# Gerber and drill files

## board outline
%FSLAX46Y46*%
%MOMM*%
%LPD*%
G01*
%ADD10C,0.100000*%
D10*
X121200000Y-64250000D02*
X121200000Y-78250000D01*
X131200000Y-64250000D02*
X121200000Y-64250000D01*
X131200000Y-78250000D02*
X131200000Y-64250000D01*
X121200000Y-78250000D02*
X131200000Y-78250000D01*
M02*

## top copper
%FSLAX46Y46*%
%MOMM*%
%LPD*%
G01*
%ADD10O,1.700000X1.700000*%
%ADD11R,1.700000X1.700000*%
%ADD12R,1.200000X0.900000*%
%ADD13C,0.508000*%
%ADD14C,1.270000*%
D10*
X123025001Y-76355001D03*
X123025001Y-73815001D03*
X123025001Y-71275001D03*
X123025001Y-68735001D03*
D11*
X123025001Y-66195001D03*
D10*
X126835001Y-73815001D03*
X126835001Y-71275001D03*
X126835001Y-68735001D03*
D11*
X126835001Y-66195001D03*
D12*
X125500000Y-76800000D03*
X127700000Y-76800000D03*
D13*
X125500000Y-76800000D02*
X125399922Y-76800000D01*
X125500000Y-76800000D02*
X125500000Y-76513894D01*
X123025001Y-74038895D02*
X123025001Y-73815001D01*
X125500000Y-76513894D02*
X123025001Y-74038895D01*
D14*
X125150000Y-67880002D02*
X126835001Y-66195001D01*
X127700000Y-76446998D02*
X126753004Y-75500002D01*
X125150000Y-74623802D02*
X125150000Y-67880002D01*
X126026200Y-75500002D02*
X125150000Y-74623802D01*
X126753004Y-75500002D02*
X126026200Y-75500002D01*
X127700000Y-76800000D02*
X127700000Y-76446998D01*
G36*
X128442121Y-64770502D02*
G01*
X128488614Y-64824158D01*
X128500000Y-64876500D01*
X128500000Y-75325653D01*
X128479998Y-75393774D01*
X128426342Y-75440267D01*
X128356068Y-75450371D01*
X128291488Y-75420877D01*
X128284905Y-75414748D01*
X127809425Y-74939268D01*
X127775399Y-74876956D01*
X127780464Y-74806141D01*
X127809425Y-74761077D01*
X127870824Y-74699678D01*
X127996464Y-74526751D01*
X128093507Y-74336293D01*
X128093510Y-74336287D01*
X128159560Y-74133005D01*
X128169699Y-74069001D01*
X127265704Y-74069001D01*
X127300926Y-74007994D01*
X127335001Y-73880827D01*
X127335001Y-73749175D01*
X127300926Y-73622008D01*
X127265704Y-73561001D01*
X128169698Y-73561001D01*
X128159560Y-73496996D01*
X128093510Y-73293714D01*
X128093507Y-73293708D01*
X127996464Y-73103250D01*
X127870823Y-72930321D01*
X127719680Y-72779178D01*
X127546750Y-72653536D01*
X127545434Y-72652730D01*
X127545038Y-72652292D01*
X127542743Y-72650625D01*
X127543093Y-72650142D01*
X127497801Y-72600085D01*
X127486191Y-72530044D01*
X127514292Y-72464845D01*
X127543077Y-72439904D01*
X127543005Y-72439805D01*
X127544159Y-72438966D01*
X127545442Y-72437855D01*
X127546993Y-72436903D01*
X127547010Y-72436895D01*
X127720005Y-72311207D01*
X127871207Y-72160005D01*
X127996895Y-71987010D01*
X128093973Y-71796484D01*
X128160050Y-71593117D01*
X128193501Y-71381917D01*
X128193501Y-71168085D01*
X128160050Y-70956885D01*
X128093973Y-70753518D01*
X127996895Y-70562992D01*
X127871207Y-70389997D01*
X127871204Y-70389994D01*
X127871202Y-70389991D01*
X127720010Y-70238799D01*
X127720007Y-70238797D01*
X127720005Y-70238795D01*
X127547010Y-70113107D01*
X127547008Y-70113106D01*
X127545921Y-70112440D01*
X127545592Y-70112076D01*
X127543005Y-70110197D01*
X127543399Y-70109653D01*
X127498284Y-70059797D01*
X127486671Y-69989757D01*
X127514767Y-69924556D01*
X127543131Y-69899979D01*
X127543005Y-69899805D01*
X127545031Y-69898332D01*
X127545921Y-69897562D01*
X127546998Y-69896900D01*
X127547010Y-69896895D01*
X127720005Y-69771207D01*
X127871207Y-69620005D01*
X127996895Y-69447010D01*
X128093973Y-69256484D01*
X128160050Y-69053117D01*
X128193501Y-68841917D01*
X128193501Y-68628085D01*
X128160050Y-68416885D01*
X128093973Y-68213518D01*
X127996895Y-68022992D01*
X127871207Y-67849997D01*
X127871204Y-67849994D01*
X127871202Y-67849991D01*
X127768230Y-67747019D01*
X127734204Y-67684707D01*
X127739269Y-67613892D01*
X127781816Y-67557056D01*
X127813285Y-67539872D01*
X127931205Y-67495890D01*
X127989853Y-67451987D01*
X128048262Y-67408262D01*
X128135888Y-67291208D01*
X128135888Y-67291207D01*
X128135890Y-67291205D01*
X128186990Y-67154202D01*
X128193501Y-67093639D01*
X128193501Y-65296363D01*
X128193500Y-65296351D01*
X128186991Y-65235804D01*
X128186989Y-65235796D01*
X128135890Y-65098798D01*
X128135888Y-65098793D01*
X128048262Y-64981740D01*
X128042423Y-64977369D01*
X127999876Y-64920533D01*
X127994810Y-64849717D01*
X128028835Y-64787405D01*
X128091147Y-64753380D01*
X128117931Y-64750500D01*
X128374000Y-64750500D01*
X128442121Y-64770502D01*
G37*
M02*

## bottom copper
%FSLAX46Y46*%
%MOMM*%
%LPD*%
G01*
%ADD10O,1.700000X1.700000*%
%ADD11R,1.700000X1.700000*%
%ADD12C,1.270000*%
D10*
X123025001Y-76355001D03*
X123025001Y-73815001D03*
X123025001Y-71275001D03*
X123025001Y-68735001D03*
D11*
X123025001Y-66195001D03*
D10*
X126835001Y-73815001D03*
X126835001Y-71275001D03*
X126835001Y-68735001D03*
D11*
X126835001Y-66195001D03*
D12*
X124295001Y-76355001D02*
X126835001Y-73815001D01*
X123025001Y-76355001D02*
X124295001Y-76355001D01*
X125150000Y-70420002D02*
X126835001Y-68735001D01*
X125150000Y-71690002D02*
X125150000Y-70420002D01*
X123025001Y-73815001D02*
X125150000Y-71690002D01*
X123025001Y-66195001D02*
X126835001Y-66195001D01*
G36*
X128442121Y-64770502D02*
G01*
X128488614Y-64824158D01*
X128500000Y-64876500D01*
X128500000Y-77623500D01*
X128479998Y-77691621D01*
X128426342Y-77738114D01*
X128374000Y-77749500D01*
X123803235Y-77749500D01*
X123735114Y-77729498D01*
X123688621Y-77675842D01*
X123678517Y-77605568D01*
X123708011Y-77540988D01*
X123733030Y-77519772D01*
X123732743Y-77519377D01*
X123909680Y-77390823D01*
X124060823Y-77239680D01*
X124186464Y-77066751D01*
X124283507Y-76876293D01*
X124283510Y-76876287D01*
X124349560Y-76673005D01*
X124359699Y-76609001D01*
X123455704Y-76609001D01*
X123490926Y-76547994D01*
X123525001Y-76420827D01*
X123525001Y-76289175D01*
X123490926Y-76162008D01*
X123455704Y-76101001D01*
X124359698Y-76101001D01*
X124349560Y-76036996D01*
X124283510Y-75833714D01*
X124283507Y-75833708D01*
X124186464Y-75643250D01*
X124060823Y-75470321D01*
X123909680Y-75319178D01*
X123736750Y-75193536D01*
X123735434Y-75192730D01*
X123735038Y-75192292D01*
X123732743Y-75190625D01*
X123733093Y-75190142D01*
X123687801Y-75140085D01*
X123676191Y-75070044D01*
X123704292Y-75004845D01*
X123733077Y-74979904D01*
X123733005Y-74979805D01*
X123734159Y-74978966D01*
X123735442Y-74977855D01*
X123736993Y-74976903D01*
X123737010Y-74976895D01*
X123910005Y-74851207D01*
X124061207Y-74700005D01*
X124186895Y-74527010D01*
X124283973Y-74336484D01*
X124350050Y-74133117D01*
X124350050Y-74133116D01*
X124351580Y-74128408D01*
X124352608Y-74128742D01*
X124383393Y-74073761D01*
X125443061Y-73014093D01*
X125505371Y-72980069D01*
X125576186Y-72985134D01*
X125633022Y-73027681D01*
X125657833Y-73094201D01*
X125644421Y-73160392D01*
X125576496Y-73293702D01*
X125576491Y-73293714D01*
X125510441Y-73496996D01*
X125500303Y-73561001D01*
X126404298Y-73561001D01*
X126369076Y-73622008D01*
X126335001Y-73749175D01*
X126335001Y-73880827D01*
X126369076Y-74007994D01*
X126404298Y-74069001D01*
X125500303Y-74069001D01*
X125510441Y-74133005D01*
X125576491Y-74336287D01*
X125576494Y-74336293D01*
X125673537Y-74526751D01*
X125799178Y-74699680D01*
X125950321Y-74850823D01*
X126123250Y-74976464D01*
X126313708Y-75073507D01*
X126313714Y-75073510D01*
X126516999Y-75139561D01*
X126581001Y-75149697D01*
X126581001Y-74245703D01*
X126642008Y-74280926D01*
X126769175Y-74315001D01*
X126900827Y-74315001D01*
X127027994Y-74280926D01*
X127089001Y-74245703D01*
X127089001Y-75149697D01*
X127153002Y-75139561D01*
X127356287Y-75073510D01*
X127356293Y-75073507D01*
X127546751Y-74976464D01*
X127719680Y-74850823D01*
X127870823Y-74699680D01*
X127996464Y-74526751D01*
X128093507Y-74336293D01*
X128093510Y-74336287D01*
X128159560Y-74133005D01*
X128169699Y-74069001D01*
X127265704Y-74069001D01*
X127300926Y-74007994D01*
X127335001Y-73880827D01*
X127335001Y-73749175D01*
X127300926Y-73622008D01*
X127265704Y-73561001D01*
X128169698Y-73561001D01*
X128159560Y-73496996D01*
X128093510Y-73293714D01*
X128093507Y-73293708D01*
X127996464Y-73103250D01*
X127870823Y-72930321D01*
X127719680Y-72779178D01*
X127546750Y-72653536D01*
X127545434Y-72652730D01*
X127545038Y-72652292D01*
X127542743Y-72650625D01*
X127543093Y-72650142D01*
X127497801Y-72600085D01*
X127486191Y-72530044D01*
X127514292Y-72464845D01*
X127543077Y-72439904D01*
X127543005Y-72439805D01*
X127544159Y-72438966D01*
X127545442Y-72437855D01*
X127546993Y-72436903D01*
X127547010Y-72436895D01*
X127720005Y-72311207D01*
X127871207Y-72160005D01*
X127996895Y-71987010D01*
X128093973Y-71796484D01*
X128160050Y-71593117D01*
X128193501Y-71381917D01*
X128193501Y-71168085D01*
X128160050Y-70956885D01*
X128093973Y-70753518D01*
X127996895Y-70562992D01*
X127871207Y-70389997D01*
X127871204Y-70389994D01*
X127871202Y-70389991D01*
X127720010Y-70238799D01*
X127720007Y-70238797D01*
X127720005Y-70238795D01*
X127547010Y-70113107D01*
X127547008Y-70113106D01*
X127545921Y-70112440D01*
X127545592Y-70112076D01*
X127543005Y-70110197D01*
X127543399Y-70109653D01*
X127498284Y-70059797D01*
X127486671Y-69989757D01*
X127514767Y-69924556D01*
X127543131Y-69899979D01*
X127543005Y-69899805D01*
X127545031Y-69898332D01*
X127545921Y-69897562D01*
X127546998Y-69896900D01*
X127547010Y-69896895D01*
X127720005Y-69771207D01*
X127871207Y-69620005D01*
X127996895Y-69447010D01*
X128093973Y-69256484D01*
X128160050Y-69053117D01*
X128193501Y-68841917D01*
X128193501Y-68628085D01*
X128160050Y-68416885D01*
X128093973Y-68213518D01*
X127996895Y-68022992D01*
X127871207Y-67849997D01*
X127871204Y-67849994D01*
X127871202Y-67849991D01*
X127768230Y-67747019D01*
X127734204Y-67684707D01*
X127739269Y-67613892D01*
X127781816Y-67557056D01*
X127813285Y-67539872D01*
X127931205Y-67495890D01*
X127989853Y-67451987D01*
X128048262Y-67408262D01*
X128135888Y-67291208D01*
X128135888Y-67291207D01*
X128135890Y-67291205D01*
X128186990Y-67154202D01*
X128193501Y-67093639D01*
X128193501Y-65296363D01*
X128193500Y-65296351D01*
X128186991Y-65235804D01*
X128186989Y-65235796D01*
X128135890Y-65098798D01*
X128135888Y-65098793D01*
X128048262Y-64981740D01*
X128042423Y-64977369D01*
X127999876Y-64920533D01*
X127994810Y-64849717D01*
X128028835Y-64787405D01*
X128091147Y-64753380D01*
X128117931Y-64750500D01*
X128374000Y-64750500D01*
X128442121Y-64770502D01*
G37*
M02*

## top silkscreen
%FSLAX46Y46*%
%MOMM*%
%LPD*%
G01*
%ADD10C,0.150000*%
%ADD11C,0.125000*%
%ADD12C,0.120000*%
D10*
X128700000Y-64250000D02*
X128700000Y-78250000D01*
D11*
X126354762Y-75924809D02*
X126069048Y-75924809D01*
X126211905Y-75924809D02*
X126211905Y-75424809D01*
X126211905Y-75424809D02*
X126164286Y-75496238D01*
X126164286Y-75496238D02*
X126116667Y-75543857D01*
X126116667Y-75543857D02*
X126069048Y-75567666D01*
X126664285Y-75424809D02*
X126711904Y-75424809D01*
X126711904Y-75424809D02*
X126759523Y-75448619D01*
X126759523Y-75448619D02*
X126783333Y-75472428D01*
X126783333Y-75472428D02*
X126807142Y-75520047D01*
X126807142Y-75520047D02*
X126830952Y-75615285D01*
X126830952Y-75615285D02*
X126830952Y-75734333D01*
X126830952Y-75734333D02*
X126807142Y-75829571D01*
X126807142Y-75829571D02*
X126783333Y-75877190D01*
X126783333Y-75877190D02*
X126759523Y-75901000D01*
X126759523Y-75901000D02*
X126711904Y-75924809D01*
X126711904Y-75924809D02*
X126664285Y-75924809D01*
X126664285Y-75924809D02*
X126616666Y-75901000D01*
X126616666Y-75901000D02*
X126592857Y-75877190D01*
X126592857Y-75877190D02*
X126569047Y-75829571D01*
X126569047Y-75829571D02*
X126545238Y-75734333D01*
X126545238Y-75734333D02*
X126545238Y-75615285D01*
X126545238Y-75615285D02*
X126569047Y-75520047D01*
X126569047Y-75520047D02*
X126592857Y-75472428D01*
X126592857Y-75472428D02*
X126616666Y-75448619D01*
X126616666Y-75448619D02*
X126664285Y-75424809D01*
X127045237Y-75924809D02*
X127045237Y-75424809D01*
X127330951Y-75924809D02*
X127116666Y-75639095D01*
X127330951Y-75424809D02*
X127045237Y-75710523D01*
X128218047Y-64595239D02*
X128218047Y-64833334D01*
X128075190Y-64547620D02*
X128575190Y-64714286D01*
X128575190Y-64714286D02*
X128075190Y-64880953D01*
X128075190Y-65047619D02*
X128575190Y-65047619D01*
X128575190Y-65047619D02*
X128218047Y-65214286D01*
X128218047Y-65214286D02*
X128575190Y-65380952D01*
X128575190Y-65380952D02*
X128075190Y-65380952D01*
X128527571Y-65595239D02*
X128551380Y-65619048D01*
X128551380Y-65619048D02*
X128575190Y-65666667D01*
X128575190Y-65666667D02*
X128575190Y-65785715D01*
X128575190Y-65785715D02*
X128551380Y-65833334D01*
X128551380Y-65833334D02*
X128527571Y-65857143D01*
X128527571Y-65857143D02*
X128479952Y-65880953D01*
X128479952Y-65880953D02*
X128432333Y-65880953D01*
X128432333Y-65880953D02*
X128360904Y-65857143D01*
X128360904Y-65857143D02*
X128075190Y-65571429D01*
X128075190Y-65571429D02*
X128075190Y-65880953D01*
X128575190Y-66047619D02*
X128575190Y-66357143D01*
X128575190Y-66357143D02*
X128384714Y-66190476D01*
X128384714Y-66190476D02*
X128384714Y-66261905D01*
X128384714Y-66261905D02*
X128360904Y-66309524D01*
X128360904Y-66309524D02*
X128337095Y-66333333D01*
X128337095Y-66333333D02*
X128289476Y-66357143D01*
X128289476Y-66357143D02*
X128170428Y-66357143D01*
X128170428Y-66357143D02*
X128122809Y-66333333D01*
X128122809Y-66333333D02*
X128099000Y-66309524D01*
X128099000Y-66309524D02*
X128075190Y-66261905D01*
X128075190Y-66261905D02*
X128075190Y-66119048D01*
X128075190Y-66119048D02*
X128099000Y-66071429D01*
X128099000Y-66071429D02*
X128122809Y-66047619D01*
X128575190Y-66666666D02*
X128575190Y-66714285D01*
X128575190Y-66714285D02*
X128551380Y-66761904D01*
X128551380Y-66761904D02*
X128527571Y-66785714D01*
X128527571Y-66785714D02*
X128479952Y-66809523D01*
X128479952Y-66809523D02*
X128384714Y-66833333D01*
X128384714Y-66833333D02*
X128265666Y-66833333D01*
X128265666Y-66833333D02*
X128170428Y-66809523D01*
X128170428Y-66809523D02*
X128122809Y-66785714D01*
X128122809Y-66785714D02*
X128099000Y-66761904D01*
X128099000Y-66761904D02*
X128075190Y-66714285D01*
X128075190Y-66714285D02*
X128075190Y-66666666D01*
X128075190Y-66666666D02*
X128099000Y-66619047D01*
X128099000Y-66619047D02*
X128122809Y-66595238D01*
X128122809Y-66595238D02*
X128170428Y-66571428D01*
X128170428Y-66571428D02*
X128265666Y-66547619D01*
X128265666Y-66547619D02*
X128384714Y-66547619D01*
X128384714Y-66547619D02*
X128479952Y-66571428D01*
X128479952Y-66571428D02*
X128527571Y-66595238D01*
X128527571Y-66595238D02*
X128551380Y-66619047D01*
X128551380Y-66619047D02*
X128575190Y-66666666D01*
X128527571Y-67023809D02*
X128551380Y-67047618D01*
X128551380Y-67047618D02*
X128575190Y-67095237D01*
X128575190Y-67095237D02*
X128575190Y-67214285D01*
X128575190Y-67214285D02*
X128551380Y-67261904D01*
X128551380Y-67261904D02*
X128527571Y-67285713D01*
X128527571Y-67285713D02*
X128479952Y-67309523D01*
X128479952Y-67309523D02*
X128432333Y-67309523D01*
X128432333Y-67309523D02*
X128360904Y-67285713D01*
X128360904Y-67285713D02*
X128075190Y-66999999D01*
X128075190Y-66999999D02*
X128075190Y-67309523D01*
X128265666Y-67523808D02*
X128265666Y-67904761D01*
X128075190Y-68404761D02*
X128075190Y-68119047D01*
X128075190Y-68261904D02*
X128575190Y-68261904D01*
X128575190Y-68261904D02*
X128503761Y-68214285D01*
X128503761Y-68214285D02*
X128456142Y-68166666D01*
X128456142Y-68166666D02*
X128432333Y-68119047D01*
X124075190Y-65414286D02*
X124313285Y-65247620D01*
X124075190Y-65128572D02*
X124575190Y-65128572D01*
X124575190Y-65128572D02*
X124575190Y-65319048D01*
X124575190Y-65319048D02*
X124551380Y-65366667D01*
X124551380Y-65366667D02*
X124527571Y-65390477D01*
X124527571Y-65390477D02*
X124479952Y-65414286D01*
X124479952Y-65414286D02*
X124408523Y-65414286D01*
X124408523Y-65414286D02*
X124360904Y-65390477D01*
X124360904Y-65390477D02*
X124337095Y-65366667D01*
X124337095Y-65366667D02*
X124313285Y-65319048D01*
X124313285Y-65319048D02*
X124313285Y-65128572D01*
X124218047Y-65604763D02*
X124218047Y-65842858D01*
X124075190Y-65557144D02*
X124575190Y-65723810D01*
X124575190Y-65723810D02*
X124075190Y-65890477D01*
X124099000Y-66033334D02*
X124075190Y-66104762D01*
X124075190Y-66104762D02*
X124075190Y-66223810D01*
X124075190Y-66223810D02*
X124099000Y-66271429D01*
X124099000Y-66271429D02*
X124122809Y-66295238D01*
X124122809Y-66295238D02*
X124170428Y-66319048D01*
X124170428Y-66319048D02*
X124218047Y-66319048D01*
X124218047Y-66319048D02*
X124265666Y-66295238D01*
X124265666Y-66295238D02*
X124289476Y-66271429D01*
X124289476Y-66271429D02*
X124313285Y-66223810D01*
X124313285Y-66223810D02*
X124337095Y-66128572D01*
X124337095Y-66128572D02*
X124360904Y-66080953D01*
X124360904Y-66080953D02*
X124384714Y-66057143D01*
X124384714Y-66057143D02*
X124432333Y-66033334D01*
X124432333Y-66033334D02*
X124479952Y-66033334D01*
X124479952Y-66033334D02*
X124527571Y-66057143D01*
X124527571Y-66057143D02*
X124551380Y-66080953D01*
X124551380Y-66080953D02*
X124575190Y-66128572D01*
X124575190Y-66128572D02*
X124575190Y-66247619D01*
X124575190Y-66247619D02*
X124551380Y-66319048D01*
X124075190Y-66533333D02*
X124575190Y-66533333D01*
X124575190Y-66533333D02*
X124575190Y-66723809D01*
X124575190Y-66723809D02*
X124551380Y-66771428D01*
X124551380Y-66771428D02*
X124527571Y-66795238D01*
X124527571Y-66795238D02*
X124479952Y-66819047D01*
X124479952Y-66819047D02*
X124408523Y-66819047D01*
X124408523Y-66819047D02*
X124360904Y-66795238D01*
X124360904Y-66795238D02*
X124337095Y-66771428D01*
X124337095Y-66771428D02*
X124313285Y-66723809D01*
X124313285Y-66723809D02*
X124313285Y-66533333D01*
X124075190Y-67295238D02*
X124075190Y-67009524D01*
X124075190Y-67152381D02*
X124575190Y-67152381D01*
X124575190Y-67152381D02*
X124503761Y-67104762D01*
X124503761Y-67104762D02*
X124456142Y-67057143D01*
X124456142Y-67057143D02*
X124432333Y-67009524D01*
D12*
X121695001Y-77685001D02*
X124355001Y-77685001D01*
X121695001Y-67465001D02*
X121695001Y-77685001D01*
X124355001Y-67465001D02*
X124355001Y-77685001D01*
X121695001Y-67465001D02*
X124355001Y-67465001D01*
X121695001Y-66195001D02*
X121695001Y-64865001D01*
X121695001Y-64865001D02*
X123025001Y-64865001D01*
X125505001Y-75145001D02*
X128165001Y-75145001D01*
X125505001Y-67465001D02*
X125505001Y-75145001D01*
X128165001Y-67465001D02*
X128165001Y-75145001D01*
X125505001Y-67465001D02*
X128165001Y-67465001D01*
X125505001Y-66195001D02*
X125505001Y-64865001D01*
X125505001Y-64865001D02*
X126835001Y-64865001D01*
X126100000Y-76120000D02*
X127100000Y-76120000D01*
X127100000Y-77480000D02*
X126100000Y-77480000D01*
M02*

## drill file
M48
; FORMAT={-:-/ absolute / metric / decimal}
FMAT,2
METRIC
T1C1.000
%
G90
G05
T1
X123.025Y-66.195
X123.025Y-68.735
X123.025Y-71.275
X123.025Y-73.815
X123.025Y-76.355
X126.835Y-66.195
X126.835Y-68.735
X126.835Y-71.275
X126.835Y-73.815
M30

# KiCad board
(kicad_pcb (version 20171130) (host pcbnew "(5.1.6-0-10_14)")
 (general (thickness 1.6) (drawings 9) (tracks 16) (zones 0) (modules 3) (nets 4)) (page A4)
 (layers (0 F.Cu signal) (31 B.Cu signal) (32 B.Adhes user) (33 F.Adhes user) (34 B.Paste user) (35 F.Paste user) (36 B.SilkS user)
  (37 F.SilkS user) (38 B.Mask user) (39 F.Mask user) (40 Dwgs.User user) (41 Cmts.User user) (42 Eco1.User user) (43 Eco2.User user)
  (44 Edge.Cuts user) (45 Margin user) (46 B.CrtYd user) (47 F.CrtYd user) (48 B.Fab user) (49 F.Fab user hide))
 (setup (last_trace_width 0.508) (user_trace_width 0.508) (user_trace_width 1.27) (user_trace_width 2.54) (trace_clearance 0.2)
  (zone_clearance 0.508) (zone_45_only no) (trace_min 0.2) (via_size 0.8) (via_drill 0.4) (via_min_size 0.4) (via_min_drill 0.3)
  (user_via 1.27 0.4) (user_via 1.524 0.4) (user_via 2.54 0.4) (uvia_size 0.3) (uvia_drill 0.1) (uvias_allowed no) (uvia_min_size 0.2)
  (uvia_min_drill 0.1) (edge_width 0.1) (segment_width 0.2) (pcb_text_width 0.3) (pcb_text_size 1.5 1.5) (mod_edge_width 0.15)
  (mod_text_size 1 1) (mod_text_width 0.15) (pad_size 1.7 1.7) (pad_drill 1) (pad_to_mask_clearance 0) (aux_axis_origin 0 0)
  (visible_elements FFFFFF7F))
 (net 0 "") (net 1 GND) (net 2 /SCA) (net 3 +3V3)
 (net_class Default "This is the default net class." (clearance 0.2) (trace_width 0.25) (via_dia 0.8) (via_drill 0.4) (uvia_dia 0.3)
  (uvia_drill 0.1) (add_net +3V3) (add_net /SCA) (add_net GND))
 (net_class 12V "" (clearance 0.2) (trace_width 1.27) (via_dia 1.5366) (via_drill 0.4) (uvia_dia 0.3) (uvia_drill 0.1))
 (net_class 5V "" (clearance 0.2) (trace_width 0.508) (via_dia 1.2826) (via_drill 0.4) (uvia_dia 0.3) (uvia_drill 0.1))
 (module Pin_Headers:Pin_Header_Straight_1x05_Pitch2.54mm (layer F.Cu) (at 123.025001 66.195001)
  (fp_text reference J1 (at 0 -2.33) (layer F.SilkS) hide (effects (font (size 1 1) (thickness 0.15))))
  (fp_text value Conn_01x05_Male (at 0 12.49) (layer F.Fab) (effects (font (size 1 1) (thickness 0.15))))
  (fp_line (start -1.33 11.49) (end 1.33 11.49) (layer F.SilkS) (width 0.12))
  (fp_line (start -1.33 1.27) (end -1.33 11.49) (layer F.SilkS) (width 0.12))
  (fp_line (start 1.33 1.27) (end 1.33 11.49) (layer F.SilkS) (width 0.12))
  (fp_line (start -1.33 1.27) (end 1.33 1.27) (layer F.SilkS) (width 0.12))
  (fp_line (start -1.33 0) (end -1.33 -1.33) (layer F.SilkS) (width 0.12))
  (fp_line (start -1.33 -1.33) (end 0 -1.33) (layer F.SilkS) (width 0.12))
  (pad 5 thru_hole oval (at 0 10.16) (size 1.7 1.7) (drill 1) (layers *.Cu *.Mask) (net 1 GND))
  (pad 4 thru_hole oval (at 0 7.62) (size 1.7 1.7) (drill 1) (layers *.Cu *.Mask) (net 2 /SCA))
  (pad 3 thru_hole oval (at 0 5.08) (size 1.7 1.7) (drill 1) (layers *.Cu *.Mask))
  (pad 2 thru_hole oval (at 0 2.54) (size 1.7 1.7) (drill 1) (layers *.Cu *.Mask))
  (pad 1 thru_hole rect (at 0 0) (size 1.7 1.7) (drill 1) (layers *.Cu *.Mask) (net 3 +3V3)))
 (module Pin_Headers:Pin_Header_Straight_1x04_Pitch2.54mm (layer F.Cu) (at 126.835001 66.195001)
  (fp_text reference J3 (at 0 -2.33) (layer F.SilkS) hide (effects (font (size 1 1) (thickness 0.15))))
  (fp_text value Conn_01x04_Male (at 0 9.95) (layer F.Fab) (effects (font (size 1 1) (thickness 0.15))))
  (fp_line (start -1.33 8.95) (end 1.33 8.95) (layer F.SilkS) (width 0.12))
  (fp_line (start -1.33 1.27) (end -1.33 8.95) (layer F.SilkS) (width 0.12))
  (fp_line (start 1.33 1.27) (end 1.33 8.95) (layer F.SilkS) (width 0.12))
  (fp_line (start -1.33 1.27) (end 1.33 1.27) (layer F.SilkS) (width 0.12))
  (fp_line (start -1.33 0) (end -1.33 -1.33) (layer F.SilkS) (width 0.12))
  (fp_line (start -1.33 -1.33) (end 0 -1.33) (layer F.SilkS) (width 0.12))
  (pad 4 thru_hole oval (at 0 7.62) (size 1.7 1.7) (drill 1) (layers *.Cu *.Mask) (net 1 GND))
  (pad 3 thru_hole oval (at 0 5.08) (size 1.7 1.7) (drill 1) (layers *.Cu *.Mask))
  (pad 2 thru_hole oval (at 0 2.54) (size 1.7 1.7) (drill 1) (layers *.Cu *.Mask) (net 2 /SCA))
  (pad 1 thru_hole rect (at 0 0) (size 1.7 1.7) (drill 1) (layers *.Cu *.Mask) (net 3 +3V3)))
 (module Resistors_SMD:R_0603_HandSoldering (layer F.Cu) (at 126.6 76.8 180)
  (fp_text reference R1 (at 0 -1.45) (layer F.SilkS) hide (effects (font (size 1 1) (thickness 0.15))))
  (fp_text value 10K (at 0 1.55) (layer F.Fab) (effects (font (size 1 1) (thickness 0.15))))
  (fp_line (start 0.5 0.68) (end -0.5 0.68) (layer F.SilkS) (width 0.12))
  (fp_line (start -0.5 -0.68) (end 0.5 -0.68) (layer F.SilkS) (width 0.12))
  (pad 2 smd rect (at 1.1 0 180) (size 1.2 0.9) (layers F.Cu F.Paste F.Mask) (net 2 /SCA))
  (pad 1 smd rect (at -1.1 0 180) (size 1.2 0.9) (layers F.Cu F.Paste F.Mask) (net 3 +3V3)))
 (gr_line (start 128.7 64.25) (end 128.7 78.25) (layer F.SilkS) (width 0.15))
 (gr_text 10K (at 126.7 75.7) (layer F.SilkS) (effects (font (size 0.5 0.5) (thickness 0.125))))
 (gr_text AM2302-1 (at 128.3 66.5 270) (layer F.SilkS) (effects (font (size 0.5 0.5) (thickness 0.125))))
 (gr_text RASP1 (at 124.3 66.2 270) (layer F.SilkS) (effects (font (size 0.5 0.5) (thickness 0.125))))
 (gr_line (start 121.2 64.25) (end 121.2 78.25) (layer Edge.Cuts) (width 0.1))
 (gr_line (start 131.2 64.25) (end 121.2 64.25) (layer Edge.Cuts) (width 0.1))
 (gr_line (start 131.2 78.25) (end 131.2 64.25) (layer Edge.Cuts) (width 0.1))
 (gr_line (start 121.2 78.25) (end 131.2 78.25) (layer Edge.Cuts) (width 0.1))
 (segment (start 124.295001 76.355001) (end 126.835001 73.815001) (width 1.27) (layer B.Cu) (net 1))
 (segment (start 123.025001 76.355001) (end 124.295001 76.355001) (width 1.27) (layer B.Cu) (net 1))
 (segment (start 125.15 70.420002) (end 126.835001 68.735001) (width 1.27) (layer B.Cu) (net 2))
 (segment (start 125.15 71.690002) (end 125.15 70.420002) (width 1.27) (layer B.Cu) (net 2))
 (segment (start 123.025001 73.815001) (end 125.15 71.690002) (width 1.27) (layer B.Cu) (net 2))
 (segment (start 125.5 76.8) (end 125.399922 76.8) (width 0.508) (layer F.Cu) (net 2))
 (segment (start 125.5 76.8) (end 125.5 76.513894) (width 0.508) (layer F.Cu) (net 2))
 (segment (start 123.025001 74.038895) (end 123.025001 73.815001) (width 0.508) (layer F.Cu) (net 2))
 (segment (start 125.5 76.513894) (end 123.025001 74.038895) (width 0.508) (layer F.Cu) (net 2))
 (segment (start 123.025001 66.195001) (end 126.835001 66.195001) (width 1.27) (layer B.Cu) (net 3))
 (segment (start 125.15 67.880002) (end 126.835001 66.195001) (width 1.27) (layer F.Cu) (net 3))
 (segment (start 127.7 76.446998) (end 126.753004 75.500002) (width 1.27) (layer F.Cu) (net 3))
 (segment (start 125.15 74.623802) (end 125.15 67.880002) (width 1.27) (layer F.Cu) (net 3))
 (segment (start 126.0262 75.500002) (end 125.15 74.623802) (width 1.27) (layer F.Cu) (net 3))
 (segment (start 126.753004 75.500002) (end 126.0262 75.500002) (width 1.27) (layer F.Cu) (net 3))
 (segment (start 127.7 76.8) (end 127.7 76.446998) (width 1.27) (layer F.Cu) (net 3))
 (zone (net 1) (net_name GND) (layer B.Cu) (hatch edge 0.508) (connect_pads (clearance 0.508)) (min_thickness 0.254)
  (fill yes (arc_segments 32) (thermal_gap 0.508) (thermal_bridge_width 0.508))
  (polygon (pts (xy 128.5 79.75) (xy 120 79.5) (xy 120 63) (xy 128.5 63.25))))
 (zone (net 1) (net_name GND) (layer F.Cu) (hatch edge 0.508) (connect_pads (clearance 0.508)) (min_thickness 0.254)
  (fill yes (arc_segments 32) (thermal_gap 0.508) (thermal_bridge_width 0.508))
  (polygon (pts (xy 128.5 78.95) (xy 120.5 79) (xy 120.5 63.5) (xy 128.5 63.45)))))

